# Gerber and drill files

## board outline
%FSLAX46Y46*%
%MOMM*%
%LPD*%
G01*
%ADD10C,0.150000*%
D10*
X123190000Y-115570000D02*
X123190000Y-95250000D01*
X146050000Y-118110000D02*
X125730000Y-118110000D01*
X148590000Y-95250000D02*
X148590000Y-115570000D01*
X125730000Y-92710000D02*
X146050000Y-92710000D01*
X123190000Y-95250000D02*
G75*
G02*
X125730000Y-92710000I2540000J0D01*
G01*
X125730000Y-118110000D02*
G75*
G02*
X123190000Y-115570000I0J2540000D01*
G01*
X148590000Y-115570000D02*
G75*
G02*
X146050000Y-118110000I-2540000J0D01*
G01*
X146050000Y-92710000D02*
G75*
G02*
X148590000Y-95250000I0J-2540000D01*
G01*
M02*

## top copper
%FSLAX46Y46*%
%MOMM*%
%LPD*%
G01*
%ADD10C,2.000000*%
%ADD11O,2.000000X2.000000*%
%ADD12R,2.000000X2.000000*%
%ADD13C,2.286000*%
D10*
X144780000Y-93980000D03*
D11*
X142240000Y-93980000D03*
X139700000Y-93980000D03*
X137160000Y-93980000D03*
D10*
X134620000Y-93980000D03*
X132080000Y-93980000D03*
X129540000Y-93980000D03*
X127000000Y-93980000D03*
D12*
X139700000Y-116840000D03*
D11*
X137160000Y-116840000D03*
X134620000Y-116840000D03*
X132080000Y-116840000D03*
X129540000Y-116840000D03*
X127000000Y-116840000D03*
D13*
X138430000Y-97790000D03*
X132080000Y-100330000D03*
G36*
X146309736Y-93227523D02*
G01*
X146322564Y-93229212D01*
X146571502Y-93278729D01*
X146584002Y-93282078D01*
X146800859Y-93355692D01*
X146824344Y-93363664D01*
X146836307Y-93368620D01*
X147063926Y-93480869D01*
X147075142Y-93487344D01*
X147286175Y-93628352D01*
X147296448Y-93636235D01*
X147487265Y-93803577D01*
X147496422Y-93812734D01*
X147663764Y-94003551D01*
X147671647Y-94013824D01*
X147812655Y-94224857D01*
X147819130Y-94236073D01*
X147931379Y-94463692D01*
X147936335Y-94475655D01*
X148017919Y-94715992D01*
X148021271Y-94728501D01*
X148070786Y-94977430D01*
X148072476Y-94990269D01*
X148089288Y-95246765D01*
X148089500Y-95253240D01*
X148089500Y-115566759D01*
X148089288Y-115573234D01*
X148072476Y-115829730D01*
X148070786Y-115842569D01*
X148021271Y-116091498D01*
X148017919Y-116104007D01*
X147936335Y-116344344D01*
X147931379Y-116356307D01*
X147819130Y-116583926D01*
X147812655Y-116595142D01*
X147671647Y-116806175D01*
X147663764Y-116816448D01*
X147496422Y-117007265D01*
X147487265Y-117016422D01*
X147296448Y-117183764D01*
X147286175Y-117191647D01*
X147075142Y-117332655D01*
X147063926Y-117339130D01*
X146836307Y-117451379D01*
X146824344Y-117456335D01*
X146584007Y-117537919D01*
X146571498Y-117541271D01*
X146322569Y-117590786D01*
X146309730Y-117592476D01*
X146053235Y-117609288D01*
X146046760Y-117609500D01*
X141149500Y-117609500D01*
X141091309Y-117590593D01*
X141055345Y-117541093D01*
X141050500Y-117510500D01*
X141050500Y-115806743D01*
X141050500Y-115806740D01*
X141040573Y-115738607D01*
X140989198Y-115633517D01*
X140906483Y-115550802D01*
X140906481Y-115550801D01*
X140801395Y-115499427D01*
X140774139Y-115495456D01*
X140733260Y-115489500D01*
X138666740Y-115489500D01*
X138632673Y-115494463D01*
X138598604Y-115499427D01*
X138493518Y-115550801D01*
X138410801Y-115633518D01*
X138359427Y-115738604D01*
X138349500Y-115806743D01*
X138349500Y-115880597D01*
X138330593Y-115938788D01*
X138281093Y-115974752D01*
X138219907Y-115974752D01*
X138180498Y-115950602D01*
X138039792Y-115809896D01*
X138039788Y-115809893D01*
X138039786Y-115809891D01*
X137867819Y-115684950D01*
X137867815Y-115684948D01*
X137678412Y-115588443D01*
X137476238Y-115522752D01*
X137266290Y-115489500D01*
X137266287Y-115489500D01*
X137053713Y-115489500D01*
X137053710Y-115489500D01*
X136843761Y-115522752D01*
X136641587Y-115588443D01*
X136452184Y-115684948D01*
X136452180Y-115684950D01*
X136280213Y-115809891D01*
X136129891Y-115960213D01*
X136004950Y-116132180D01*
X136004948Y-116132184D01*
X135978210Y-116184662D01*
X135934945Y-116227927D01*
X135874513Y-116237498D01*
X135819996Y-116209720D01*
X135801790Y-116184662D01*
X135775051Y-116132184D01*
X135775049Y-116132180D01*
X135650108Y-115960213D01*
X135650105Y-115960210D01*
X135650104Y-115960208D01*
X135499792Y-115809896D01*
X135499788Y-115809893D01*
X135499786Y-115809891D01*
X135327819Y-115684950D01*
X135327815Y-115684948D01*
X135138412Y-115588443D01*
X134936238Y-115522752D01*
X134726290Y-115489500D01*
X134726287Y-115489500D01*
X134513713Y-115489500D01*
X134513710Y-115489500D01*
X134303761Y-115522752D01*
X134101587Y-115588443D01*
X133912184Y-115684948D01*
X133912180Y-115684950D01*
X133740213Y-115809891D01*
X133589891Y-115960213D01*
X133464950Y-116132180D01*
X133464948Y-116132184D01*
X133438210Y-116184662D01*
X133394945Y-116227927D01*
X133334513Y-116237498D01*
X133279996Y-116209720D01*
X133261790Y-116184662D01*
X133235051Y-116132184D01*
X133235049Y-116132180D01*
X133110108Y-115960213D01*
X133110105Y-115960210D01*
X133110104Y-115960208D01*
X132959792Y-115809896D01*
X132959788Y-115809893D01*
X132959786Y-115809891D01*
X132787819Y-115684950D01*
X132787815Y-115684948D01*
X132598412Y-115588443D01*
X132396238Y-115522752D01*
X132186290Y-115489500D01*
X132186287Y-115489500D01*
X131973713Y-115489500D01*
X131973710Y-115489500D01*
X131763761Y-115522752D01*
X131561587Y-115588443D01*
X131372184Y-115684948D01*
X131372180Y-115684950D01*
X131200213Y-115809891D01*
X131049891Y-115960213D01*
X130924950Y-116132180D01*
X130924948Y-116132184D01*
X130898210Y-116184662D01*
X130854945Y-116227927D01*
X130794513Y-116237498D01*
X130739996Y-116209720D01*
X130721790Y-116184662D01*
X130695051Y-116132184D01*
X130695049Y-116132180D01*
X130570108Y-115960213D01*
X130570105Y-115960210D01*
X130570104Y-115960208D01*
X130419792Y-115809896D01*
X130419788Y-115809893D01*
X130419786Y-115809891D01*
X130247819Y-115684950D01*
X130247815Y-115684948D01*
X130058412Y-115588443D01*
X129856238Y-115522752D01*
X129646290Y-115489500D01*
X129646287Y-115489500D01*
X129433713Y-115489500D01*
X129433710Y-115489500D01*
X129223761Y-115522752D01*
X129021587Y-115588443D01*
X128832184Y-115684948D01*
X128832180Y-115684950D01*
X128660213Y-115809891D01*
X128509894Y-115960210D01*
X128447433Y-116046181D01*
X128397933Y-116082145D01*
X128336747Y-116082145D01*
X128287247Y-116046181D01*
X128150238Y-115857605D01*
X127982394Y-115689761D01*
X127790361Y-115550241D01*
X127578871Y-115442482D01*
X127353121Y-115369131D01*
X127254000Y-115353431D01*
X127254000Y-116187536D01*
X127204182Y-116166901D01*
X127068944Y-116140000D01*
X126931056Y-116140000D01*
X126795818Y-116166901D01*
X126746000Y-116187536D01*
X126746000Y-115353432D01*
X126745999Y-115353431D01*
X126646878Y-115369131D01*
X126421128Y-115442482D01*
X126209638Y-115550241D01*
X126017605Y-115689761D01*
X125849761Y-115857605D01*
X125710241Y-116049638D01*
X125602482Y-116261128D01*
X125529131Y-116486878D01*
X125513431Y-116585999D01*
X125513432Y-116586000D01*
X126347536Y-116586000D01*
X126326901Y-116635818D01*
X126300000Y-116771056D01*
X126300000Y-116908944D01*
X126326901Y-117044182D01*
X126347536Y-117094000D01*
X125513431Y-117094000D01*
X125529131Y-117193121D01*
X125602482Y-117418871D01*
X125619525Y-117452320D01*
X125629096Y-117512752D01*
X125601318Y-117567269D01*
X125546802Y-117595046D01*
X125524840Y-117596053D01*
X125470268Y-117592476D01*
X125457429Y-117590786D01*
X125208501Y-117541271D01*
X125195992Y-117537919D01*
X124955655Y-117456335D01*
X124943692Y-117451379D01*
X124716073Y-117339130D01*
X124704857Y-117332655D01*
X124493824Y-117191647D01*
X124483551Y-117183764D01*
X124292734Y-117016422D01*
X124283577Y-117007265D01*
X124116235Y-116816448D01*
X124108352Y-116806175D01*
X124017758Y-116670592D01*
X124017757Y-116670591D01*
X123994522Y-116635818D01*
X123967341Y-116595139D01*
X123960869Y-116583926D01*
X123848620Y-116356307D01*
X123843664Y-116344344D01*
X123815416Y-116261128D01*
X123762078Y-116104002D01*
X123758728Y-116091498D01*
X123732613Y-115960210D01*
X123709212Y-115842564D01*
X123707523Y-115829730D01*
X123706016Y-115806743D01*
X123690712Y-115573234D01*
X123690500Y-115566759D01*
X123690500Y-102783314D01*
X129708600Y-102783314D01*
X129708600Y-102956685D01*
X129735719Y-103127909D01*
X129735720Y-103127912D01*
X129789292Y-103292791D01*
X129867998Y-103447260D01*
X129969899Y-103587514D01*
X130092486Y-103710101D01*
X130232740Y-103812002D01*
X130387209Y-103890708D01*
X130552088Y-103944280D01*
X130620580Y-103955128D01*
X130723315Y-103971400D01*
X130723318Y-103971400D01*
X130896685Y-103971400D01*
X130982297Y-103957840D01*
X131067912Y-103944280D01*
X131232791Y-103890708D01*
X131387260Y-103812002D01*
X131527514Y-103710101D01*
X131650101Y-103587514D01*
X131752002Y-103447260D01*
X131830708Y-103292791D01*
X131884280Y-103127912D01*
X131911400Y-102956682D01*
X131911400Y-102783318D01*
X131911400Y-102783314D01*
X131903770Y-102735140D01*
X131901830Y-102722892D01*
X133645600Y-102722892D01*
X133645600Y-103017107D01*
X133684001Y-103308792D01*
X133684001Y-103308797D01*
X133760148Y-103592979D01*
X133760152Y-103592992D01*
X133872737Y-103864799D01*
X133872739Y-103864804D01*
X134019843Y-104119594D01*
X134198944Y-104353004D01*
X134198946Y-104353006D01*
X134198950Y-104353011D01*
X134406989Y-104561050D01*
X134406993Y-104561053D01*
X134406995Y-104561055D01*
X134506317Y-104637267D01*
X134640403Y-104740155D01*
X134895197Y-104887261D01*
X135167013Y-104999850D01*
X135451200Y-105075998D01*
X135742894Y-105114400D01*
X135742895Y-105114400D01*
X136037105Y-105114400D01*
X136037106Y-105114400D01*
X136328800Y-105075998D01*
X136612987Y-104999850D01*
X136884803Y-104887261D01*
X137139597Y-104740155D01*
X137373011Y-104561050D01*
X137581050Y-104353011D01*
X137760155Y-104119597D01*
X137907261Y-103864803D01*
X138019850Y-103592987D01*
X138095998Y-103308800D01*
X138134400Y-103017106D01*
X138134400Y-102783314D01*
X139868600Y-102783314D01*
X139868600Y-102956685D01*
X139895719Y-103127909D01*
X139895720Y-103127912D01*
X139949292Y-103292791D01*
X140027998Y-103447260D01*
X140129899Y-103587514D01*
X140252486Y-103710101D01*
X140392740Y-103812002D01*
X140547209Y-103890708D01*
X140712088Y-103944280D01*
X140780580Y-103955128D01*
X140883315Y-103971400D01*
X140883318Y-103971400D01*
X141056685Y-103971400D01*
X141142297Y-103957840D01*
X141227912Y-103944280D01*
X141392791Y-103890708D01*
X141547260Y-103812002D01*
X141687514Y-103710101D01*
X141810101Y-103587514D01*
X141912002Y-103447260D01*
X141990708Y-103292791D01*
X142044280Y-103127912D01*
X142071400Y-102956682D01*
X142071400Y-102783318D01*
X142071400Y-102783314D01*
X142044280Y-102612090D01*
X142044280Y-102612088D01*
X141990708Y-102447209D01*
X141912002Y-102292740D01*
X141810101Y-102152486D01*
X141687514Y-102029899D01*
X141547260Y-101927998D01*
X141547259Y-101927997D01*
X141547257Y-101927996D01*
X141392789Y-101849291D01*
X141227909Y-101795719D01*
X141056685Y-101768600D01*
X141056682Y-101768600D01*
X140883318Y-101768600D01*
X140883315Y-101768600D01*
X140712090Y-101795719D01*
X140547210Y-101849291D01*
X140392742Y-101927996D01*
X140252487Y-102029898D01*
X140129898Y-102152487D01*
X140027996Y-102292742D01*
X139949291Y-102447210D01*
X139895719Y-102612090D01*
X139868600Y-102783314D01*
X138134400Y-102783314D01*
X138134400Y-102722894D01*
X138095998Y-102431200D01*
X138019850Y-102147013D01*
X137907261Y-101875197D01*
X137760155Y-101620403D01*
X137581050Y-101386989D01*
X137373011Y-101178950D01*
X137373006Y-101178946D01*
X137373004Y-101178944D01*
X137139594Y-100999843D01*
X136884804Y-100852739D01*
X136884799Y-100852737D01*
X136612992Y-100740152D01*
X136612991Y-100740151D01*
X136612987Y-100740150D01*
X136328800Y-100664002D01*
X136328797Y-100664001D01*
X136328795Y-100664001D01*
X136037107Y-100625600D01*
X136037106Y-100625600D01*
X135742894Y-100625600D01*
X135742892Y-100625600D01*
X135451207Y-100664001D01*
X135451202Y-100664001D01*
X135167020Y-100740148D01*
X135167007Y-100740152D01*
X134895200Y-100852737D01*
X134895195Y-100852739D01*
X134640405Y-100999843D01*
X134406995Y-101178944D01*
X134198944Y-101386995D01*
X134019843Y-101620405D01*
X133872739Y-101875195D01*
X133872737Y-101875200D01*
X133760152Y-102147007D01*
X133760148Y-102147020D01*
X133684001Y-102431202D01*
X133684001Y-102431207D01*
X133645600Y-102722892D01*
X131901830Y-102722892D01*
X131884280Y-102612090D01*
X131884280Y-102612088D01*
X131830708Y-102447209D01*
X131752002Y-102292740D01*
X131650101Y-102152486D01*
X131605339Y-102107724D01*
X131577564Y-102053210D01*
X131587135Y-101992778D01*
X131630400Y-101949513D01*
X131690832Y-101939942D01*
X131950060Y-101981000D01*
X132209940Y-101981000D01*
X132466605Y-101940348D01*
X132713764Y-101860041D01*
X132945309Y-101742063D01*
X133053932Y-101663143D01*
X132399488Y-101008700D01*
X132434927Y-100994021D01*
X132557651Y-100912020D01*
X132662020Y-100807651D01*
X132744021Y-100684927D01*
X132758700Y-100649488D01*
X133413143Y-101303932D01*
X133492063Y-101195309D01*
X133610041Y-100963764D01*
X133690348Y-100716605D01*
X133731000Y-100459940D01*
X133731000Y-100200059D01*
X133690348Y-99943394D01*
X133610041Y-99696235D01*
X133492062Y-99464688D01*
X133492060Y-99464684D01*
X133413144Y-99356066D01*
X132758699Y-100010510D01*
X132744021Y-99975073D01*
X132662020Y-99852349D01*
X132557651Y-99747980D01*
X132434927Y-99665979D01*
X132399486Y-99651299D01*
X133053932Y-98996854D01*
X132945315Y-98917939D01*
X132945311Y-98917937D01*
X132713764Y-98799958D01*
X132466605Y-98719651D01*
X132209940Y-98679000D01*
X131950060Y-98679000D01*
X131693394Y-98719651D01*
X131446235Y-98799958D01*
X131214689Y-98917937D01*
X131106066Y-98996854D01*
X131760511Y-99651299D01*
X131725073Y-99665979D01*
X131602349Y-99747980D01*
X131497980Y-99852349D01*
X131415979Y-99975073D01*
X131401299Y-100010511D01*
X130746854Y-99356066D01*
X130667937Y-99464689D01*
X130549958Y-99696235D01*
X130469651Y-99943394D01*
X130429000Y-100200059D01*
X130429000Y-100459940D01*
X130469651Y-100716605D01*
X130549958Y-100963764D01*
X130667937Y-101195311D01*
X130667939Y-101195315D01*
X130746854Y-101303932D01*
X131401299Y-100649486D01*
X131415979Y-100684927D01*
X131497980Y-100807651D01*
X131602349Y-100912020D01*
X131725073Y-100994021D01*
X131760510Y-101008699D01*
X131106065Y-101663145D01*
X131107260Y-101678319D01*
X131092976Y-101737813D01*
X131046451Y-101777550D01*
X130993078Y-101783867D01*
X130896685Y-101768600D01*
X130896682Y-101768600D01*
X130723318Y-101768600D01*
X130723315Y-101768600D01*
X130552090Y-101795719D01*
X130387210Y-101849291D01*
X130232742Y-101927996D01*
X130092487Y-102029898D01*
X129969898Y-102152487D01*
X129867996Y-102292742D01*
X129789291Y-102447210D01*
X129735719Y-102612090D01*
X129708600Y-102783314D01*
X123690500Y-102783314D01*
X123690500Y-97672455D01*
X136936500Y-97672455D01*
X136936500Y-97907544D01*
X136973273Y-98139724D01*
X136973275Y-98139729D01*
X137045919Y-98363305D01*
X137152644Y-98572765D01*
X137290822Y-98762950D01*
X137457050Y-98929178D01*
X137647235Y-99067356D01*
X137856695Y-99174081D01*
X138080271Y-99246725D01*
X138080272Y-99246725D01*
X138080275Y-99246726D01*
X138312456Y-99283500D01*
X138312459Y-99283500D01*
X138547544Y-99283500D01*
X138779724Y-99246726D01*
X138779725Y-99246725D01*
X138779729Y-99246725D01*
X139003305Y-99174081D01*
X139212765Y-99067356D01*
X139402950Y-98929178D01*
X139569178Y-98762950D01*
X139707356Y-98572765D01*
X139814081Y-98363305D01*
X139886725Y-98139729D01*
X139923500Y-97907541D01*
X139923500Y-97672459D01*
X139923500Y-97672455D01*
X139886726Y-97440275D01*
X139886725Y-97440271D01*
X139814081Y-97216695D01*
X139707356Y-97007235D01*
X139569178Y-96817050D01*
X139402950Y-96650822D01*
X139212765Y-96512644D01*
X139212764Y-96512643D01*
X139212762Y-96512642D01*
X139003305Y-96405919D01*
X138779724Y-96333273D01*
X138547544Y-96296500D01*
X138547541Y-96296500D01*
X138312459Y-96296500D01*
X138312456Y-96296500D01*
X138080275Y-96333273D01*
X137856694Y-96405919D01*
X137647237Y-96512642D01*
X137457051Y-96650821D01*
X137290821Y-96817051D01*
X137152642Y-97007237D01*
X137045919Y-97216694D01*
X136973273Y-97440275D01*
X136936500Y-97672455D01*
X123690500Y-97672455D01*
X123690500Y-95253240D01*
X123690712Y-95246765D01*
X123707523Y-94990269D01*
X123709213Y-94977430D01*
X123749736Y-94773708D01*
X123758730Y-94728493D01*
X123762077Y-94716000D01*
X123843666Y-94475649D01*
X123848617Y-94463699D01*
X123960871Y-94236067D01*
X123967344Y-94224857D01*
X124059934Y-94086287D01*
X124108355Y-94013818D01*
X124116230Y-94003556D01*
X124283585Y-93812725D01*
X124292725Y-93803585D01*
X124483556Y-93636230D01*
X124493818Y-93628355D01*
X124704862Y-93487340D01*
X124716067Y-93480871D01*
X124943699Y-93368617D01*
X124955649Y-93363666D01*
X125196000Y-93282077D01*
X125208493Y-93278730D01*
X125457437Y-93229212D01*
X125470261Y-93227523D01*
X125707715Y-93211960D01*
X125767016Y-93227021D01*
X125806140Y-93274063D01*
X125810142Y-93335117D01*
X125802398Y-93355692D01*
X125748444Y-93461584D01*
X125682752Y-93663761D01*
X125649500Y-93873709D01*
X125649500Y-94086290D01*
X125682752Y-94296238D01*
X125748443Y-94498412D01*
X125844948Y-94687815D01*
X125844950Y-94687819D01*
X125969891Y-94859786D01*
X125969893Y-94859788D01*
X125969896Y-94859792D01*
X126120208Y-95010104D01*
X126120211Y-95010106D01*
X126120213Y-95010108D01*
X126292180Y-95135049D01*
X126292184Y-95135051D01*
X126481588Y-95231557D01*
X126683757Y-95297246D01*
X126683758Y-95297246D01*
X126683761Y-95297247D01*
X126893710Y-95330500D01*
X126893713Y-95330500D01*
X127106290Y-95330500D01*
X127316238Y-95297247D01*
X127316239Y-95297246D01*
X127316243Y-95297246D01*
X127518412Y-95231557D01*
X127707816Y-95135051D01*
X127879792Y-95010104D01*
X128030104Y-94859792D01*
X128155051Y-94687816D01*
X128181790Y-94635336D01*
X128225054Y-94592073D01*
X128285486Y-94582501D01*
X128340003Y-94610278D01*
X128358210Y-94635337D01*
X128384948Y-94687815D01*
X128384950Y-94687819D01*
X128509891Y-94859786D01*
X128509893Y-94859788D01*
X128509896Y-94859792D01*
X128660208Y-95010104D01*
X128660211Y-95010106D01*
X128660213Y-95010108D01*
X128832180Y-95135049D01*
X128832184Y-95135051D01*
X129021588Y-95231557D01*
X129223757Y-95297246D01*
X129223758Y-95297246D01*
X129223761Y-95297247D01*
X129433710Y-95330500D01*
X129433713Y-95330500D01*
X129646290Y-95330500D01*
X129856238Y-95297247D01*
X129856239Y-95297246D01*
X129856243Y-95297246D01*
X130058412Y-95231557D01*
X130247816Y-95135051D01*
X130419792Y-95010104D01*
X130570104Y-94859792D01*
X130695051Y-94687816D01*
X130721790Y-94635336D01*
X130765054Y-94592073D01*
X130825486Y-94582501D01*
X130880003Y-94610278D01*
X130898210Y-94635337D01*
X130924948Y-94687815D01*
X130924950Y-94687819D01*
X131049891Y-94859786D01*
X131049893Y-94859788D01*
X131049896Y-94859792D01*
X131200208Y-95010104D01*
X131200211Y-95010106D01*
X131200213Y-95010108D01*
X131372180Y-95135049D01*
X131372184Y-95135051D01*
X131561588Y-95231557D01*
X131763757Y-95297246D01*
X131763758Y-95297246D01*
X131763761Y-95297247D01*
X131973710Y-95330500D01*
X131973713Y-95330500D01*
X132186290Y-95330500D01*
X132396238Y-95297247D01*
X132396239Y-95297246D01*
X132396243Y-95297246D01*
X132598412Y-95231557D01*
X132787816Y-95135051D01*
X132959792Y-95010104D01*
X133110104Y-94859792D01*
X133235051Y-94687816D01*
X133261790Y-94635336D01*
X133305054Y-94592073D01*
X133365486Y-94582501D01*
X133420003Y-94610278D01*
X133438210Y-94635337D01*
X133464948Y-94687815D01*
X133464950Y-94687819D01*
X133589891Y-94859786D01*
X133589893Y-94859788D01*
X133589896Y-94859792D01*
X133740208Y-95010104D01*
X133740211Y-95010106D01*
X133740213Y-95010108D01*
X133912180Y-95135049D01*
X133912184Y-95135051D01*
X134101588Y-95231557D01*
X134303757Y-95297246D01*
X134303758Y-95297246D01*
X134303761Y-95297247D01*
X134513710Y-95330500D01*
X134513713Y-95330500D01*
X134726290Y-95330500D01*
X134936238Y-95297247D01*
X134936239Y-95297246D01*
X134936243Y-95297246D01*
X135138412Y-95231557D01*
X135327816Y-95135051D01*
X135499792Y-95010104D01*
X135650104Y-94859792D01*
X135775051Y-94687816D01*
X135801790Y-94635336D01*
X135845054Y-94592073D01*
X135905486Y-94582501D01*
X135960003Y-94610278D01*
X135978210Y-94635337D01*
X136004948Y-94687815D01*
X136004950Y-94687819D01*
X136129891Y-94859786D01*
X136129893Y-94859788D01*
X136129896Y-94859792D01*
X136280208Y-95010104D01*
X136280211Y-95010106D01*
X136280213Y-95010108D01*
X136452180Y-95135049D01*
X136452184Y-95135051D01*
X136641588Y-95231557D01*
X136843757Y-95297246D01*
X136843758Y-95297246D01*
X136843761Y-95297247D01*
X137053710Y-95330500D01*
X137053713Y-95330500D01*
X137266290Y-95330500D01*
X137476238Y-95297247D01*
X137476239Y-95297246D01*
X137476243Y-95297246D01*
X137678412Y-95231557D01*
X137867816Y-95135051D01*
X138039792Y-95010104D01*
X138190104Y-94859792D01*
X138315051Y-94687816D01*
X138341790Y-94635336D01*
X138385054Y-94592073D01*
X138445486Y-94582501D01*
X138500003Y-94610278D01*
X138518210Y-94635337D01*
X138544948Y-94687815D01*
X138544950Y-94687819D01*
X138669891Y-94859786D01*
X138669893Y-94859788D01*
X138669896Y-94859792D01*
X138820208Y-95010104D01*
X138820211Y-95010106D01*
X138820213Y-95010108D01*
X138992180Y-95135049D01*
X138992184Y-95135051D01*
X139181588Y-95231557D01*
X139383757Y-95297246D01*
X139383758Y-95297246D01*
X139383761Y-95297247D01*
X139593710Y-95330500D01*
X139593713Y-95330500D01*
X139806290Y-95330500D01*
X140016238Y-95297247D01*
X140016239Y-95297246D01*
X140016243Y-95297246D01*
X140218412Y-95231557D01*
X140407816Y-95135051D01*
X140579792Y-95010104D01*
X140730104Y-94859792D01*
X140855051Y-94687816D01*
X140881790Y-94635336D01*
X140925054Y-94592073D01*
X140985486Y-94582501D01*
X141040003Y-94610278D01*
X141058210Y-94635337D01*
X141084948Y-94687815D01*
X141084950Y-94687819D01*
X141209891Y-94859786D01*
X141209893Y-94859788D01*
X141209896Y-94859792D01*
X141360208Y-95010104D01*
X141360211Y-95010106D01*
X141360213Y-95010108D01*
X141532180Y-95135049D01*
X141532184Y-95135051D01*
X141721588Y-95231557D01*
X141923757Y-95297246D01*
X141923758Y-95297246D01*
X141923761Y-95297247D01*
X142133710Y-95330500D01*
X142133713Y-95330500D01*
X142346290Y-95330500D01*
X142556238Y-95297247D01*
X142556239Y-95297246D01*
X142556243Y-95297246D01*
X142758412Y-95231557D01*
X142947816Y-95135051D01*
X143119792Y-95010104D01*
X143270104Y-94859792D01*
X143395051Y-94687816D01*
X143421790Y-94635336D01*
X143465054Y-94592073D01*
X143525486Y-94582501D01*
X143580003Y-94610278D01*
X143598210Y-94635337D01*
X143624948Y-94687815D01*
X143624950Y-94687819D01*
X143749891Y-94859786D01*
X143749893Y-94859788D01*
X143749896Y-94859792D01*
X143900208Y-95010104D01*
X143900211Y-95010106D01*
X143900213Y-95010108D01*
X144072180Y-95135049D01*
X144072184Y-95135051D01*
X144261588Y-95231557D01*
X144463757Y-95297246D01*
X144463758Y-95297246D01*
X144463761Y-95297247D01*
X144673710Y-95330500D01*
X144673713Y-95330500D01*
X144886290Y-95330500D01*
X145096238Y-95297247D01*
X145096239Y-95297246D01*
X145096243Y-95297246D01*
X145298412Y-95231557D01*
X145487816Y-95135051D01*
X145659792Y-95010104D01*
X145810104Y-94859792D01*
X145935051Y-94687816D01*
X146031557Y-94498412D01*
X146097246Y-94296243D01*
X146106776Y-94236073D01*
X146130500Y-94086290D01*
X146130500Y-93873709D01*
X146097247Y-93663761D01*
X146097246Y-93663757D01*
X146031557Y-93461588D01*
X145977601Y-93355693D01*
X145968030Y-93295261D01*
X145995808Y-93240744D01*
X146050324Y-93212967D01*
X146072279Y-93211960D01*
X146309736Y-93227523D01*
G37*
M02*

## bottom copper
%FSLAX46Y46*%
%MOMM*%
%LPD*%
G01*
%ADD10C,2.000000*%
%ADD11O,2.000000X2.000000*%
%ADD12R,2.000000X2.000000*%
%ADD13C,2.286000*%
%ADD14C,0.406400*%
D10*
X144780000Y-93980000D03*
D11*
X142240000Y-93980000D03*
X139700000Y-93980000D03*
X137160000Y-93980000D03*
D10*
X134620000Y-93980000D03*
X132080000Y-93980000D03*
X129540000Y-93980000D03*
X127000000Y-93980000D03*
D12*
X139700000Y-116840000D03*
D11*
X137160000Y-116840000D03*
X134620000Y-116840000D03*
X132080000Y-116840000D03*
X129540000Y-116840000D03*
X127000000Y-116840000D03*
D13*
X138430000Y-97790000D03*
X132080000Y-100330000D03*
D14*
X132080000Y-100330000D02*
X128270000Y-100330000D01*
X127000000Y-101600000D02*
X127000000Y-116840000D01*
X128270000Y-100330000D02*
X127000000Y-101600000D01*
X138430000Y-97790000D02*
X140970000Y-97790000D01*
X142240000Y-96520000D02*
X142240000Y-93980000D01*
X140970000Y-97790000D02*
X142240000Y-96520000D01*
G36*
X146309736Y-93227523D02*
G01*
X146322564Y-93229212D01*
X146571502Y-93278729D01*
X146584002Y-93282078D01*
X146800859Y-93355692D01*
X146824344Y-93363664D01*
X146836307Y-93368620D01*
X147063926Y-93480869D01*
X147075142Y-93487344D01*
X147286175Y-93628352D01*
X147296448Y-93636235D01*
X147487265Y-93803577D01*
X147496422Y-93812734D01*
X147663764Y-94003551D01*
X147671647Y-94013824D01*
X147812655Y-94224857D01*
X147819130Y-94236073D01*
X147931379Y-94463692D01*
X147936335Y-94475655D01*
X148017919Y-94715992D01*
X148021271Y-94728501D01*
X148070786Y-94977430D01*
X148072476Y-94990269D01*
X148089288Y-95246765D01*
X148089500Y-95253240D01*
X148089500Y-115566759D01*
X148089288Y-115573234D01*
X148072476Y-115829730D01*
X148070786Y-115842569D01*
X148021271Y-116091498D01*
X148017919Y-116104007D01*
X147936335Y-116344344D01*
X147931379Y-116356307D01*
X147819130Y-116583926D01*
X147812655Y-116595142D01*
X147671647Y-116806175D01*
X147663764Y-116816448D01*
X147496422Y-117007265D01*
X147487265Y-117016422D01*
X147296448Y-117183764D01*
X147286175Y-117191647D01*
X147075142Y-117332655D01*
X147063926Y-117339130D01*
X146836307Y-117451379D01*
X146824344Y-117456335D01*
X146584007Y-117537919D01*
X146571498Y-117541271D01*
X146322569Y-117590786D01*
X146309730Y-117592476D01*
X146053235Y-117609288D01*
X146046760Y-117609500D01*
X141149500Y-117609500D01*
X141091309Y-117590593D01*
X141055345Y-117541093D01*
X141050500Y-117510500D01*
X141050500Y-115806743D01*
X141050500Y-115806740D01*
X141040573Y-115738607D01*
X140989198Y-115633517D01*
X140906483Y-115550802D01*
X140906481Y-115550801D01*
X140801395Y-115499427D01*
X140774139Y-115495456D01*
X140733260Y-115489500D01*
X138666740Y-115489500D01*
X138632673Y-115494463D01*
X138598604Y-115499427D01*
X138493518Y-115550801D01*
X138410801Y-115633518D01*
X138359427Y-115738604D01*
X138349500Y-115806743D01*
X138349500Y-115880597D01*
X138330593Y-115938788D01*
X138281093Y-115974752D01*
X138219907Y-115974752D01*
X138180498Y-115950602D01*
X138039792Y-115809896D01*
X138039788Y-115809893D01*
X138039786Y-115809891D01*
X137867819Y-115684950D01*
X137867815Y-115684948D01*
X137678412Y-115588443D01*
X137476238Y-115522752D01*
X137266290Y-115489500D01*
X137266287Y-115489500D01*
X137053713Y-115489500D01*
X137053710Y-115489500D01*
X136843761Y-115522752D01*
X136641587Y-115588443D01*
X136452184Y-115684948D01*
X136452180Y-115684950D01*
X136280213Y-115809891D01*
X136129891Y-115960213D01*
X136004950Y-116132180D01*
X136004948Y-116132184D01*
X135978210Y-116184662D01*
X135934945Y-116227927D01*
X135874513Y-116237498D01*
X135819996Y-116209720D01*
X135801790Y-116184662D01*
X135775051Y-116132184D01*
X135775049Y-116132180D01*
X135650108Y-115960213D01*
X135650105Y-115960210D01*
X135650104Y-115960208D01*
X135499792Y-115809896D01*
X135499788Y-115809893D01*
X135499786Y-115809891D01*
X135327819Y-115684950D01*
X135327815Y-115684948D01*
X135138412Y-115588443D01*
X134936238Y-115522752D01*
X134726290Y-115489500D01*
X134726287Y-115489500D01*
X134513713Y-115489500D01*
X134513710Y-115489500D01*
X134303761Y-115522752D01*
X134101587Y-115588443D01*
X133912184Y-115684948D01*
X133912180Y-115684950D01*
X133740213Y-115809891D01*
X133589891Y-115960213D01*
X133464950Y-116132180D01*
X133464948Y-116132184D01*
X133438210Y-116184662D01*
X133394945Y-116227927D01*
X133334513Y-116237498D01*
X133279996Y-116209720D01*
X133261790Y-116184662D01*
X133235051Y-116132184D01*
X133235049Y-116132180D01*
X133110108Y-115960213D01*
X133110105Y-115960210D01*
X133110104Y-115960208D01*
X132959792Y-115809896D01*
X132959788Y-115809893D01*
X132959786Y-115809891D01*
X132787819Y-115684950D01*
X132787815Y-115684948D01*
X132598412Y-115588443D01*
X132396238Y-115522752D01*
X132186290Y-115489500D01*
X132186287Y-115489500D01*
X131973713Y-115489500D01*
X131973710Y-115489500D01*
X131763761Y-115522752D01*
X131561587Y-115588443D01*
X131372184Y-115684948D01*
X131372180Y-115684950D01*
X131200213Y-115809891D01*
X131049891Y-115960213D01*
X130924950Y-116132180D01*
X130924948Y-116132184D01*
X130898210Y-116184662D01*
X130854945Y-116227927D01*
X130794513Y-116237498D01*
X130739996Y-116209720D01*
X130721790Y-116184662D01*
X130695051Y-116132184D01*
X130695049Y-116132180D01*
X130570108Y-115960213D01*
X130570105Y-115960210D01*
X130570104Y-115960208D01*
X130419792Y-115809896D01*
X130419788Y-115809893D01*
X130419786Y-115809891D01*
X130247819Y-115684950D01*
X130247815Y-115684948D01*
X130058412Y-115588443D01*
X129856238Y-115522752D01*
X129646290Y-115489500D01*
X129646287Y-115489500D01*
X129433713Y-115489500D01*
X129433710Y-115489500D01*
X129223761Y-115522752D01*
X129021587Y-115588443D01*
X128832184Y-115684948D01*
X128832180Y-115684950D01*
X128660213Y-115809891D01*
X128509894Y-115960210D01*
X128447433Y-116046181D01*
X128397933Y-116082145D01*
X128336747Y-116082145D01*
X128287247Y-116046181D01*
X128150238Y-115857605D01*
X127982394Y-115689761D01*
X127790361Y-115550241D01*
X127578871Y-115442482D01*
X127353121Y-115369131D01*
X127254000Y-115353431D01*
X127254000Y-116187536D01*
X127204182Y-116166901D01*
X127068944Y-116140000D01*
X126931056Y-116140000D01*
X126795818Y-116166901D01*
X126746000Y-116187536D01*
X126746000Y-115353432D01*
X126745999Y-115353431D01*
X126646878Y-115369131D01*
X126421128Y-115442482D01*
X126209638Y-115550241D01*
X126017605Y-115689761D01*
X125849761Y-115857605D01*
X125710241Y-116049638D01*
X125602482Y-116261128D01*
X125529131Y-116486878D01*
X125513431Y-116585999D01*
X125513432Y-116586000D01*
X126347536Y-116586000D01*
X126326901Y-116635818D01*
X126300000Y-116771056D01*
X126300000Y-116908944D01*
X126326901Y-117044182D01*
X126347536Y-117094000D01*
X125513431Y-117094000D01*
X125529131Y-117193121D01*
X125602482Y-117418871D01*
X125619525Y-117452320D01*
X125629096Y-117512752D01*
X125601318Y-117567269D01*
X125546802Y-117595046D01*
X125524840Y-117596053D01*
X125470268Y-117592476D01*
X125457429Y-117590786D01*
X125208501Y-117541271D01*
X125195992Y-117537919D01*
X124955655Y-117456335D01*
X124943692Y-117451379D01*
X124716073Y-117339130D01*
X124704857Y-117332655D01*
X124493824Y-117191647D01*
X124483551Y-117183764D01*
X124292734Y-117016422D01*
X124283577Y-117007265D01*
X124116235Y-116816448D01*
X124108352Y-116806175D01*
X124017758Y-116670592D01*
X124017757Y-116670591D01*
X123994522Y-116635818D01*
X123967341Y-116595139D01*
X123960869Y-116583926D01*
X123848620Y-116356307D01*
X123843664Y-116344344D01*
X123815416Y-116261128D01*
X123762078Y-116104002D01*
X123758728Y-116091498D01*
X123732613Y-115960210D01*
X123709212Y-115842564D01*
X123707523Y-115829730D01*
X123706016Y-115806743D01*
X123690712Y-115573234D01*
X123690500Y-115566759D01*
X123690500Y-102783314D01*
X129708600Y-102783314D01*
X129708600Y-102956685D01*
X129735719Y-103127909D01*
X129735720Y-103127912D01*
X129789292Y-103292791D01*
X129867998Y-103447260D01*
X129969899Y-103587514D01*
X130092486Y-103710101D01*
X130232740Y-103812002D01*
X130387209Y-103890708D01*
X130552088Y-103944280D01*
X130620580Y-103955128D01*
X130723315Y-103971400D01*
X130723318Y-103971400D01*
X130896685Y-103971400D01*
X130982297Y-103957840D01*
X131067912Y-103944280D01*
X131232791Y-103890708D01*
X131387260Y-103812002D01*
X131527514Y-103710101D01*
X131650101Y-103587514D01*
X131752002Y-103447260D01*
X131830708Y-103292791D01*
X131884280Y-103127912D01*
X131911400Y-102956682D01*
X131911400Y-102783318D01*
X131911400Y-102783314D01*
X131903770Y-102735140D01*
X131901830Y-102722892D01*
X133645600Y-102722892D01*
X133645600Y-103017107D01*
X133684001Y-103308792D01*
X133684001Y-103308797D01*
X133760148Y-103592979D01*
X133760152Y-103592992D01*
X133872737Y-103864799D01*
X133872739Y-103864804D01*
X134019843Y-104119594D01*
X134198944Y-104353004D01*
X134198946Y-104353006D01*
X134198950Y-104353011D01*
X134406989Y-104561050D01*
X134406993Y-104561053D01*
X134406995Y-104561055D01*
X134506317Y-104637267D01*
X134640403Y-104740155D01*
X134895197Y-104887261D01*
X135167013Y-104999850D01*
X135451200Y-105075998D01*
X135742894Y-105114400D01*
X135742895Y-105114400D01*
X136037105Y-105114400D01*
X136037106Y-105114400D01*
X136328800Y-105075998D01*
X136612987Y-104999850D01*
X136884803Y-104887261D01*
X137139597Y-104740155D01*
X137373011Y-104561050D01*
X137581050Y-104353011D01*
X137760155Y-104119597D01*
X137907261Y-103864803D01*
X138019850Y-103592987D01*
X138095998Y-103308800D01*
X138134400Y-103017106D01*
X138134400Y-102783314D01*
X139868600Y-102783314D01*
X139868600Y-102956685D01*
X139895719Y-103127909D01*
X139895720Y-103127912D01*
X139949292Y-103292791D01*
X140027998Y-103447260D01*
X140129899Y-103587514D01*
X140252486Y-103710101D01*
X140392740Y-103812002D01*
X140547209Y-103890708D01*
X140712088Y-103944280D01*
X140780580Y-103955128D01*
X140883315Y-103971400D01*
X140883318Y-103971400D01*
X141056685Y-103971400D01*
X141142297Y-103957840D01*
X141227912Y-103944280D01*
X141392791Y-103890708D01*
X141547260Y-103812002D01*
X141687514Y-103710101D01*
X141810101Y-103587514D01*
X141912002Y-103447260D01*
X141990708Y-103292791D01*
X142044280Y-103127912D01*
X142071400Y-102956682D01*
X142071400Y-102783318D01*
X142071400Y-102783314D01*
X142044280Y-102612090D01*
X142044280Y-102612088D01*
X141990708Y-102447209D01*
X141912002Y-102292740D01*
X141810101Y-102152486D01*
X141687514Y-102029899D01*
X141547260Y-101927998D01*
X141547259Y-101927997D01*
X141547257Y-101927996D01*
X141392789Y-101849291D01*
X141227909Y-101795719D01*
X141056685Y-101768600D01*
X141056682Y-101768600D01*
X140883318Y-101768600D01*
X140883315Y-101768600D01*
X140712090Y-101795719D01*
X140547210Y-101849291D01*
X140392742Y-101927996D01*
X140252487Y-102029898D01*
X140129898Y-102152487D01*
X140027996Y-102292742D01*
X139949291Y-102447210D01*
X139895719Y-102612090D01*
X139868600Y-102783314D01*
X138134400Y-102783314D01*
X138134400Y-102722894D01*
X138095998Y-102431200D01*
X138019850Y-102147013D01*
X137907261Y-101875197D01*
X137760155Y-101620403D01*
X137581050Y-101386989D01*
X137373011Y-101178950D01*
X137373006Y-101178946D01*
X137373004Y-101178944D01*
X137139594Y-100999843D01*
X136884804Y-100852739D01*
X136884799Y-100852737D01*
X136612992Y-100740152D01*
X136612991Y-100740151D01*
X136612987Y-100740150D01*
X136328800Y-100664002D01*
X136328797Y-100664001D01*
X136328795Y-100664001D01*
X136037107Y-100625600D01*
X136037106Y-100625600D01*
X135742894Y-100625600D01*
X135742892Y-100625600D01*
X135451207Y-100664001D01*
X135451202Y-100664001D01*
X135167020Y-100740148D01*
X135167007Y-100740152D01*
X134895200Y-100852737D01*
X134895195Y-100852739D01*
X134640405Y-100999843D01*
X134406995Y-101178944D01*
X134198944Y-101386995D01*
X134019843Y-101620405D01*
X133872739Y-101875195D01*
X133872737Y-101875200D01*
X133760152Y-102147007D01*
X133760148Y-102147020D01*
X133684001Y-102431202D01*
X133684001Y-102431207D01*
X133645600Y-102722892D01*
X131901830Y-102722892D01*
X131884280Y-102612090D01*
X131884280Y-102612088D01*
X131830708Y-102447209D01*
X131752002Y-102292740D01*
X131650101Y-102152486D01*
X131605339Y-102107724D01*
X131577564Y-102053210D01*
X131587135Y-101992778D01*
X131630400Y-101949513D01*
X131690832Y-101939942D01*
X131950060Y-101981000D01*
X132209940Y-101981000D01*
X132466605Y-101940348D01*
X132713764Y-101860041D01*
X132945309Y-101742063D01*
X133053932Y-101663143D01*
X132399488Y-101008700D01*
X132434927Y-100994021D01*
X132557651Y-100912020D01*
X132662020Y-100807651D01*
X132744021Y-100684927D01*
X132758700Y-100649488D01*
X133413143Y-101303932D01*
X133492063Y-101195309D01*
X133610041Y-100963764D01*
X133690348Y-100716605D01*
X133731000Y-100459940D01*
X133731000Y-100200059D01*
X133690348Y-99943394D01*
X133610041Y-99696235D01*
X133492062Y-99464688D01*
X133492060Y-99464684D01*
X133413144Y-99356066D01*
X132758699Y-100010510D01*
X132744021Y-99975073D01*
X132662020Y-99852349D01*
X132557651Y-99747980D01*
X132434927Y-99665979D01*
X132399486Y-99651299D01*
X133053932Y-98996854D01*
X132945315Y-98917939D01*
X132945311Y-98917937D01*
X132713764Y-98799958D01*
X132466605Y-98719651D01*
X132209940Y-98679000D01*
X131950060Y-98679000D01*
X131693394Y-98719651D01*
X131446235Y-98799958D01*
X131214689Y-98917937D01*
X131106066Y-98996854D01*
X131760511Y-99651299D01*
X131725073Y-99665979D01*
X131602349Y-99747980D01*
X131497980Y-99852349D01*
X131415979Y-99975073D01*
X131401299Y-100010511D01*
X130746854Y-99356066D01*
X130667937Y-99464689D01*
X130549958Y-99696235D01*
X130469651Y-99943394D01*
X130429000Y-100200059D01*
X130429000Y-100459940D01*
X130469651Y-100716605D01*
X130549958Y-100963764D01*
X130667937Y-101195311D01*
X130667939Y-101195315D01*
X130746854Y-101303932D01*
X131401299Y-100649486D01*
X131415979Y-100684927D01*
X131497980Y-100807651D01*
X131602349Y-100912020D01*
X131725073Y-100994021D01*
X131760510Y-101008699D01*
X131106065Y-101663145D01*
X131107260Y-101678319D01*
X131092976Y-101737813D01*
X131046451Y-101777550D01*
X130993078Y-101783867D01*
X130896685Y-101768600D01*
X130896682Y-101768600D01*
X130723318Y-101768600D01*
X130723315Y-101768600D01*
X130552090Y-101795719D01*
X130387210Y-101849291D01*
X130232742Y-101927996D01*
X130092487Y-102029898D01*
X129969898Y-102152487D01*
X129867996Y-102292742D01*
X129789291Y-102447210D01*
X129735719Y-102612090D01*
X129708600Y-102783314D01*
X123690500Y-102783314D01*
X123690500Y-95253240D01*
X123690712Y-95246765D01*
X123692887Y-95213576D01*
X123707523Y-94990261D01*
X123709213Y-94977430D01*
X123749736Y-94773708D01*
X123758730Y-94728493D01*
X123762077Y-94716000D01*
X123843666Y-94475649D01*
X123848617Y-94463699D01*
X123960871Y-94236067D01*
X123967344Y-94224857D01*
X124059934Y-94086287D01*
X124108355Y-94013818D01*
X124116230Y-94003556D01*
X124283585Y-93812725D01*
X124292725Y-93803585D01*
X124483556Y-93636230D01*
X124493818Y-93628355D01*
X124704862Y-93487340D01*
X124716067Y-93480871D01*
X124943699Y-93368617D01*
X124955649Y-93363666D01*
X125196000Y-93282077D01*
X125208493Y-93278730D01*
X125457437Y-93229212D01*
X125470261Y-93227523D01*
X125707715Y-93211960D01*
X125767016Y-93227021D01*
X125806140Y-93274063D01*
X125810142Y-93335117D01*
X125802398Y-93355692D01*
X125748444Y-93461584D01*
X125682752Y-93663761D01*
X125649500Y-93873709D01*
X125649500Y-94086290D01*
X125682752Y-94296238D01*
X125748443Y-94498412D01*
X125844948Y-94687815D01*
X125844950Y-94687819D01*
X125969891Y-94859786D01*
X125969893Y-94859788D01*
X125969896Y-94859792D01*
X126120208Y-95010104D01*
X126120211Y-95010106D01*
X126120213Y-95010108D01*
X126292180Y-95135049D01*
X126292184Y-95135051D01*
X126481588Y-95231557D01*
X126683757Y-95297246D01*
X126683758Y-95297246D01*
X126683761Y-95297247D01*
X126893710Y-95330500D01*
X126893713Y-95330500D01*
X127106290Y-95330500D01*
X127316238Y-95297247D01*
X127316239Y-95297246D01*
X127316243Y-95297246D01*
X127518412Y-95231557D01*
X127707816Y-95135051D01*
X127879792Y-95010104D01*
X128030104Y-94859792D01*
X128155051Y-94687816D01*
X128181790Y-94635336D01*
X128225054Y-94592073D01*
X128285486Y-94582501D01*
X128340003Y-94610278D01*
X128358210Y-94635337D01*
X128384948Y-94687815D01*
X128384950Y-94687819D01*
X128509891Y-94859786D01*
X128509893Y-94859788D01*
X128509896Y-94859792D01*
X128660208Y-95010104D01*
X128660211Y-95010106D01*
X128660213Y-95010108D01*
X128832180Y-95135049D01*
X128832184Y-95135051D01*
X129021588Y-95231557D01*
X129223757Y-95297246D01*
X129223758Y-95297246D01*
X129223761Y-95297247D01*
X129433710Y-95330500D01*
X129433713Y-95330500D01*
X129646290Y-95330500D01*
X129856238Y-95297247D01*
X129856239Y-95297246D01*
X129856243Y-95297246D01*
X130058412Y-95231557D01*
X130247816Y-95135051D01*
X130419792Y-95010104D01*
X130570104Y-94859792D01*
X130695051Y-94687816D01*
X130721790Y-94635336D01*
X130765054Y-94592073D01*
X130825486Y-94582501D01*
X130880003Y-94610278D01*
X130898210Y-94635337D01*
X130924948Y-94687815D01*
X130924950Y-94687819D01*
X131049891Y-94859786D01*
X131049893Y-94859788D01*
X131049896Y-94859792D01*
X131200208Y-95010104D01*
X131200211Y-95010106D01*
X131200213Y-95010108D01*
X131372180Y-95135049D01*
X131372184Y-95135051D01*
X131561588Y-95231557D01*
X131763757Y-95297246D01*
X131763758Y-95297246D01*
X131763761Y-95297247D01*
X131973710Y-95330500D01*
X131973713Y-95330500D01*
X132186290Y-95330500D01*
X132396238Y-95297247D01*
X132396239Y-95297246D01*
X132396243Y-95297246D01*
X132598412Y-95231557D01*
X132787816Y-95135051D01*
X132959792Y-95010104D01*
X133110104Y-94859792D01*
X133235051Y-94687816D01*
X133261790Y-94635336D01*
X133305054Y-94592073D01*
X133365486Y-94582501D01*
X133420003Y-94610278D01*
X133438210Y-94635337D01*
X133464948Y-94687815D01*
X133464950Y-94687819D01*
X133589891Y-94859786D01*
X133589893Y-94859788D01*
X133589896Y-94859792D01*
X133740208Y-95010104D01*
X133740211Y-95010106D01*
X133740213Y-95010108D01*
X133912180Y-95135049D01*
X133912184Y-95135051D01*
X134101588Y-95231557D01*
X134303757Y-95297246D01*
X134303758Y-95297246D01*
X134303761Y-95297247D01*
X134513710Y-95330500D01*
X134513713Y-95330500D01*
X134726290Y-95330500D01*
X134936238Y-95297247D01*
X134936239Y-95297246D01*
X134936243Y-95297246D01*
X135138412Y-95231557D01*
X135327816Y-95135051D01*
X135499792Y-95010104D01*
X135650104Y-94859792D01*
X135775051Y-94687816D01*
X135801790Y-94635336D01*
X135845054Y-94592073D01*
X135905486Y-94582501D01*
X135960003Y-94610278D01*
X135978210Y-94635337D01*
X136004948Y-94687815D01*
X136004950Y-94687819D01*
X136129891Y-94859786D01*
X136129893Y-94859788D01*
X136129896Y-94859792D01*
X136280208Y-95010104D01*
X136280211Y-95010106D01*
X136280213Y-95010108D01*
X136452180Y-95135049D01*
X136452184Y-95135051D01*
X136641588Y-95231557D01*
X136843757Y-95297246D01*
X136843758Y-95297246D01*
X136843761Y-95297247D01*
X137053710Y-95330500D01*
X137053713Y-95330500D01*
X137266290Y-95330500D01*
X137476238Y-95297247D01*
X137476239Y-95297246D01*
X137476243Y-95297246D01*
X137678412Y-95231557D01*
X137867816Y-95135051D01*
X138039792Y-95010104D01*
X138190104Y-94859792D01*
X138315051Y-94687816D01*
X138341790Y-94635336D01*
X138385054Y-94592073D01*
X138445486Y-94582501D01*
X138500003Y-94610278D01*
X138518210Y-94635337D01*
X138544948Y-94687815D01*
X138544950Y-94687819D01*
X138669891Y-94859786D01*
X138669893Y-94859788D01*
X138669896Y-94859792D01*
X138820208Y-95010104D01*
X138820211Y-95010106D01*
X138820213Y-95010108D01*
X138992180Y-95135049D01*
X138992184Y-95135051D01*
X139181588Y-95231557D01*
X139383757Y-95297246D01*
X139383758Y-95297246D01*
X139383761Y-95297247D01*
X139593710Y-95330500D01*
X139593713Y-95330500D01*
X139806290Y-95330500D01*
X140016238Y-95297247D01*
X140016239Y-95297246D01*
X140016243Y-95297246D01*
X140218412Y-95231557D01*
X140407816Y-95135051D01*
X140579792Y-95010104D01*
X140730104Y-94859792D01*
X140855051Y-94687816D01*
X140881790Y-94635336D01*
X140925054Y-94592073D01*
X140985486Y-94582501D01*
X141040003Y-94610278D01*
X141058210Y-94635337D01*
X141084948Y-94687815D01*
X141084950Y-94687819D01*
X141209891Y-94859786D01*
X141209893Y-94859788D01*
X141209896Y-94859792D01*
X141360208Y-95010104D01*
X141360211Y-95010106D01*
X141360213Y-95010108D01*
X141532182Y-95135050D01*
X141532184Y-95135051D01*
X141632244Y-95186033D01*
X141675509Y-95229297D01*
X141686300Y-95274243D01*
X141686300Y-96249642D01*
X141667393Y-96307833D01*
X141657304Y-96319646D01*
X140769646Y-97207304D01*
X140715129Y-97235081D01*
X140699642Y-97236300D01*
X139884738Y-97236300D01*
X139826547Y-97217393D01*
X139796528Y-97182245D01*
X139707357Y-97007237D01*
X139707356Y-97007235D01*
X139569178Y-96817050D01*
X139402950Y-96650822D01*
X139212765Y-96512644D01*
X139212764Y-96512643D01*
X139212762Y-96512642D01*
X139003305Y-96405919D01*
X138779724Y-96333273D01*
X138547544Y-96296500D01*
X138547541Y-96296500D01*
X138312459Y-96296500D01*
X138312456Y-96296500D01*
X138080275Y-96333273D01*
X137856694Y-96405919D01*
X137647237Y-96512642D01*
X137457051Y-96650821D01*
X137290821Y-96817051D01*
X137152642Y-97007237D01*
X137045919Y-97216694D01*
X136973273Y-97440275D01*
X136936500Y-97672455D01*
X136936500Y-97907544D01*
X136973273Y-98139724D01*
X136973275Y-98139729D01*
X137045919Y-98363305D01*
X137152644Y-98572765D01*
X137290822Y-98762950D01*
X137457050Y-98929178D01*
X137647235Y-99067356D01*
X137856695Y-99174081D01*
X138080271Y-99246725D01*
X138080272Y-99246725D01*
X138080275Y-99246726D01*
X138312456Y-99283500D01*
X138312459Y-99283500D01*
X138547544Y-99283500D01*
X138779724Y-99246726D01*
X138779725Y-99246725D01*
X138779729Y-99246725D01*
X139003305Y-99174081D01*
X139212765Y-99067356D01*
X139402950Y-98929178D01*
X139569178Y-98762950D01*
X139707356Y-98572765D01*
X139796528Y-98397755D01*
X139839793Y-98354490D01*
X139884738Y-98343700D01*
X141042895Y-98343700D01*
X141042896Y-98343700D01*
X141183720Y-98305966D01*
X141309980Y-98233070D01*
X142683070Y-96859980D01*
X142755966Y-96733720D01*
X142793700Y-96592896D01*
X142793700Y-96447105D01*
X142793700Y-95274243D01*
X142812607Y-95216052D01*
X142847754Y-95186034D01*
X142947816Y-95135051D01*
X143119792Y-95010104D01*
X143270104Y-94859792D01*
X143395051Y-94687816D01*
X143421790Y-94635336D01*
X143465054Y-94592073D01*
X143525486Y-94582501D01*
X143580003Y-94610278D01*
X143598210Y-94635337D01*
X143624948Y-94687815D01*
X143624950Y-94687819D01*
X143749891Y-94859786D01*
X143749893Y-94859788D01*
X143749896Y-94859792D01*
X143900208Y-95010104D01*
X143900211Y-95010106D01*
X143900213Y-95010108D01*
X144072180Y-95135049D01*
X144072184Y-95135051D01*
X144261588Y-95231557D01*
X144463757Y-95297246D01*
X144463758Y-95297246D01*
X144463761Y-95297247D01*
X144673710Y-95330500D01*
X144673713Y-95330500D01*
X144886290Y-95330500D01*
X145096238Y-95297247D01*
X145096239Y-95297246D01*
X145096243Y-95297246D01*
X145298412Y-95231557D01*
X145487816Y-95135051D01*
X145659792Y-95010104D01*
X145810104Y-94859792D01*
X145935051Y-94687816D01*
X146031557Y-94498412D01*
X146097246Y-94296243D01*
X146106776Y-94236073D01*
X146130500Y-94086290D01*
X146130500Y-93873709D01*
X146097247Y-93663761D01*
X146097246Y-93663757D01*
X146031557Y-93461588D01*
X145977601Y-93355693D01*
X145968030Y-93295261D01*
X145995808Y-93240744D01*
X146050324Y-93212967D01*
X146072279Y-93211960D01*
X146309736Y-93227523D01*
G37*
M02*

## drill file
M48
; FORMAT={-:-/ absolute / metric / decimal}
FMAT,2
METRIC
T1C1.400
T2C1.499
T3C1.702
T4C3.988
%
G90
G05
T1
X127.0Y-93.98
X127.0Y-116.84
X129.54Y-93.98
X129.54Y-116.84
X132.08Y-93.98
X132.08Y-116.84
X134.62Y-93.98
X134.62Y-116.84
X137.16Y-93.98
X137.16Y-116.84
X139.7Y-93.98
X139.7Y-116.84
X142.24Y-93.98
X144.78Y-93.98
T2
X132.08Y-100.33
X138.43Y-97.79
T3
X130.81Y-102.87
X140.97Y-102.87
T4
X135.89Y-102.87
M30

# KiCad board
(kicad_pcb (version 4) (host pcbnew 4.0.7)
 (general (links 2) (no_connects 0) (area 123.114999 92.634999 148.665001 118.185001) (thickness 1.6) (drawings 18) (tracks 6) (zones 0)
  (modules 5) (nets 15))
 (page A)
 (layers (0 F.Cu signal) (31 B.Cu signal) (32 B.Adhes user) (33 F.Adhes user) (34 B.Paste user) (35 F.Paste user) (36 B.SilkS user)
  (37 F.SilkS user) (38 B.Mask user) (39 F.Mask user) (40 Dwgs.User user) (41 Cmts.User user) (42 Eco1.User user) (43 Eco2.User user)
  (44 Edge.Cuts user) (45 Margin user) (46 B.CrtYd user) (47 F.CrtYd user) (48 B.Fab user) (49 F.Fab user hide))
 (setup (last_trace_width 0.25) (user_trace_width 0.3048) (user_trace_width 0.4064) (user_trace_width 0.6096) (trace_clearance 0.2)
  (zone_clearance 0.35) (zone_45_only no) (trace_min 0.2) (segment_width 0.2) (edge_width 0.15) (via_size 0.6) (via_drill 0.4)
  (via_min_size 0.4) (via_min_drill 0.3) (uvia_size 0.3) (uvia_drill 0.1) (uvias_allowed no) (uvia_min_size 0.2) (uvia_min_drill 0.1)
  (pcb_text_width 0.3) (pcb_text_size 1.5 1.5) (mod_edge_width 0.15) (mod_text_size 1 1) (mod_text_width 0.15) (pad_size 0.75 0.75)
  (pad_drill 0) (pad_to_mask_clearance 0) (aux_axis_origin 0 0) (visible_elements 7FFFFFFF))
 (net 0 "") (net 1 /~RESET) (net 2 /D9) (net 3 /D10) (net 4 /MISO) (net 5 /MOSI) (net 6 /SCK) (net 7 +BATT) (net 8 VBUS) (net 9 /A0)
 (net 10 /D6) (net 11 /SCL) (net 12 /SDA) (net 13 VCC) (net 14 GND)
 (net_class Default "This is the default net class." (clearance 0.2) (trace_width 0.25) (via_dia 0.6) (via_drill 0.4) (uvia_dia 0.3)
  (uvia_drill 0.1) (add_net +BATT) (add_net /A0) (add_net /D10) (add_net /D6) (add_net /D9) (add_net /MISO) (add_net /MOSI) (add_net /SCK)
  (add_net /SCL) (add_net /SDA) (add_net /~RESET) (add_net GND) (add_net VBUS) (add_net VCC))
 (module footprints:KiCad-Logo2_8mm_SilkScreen (layer B.Cu) (at 139.192 109.347 180)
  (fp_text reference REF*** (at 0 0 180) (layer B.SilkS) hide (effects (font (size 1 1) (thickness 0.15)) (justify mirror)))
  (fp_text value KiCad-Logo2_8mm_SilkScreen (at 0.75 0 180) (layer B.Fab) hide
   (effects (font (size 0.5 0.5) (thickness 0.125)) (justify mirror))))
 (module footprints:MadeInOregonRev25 (layer F.Cu) (at 127 108.966)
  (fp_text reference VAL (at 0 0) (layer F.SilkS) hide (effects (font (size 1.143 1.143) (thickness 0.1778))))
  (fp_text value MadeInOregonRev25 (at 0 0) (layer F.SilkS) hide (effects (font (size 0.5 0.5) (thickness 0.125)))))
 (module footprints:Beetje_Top (layer F.Cu) (at 144.78 93.98 270)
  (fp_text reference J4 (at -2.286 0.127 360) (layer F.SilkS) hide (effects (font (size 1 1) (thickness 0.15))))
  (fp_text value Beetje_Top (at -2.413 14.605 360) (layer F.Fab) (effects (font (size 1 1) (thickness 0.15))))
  (pad 1 thru_hole circle (at 0 0 270) (size 2 2) (drill 1.4) (layers *.Cu *.Mask) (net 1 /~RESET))
  (pad 2 thru_hole oval (at 0 2.54 270) (size 2 2) (drill 1.4) (layers *.Cu *.Mask) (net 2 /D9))
  (pad 3 thru_hole oval (at 0 5.08 270) (size 2 2) (drill 1.4) (layers *.Cu *.Mask) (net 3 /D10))
  (pad 4 thru_hole oval (at 0 7.62 270) (size 2 2) (drill 1.4) (layers *.Cu *.Mask) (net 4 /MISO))
  (pad 5 thru_hole circle (at 0 10.16 270) (size 2 2) (drill 1.4) (layers *.Cu *.Mask) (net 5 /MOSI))
  (pad 6 thru_hole circle (at 0 12.7 270) (size 2 2) (drill 1.4) (layers *.Cu *.Mask) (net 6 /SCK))
  (pad 7 thru_hole circle (at 0 15.24 270) (size 2 2) (drill 1.4) (layers *.Cu *.Mask) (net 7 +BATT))
  (pad 8 thru_hole circle (at 0 17.78 270) (size 2 2) (drill 1.4) (layers *.Cu *.Mask) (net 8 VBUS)))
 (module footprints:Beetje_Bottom (layer F.Cu) (at 139.7 116.84 270)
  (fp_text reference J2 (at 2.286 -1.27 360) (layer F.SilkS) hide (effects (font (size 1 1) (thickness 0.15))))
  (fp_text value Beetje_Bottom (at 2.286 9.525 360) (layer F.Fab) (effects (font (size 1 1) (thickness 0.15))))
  (pad 1 thru_hole rect (at 0 0 270) (size 2 2) (drill 1.4) (layers *.Cu *.Mask) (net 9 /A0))
  (pad 2 thru_hole oval (at 0 2.54 270) (size 2 2) (drill 1.4) (layers *.Cu *.Mask) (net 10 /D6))
  (pad 3 thru_hole oval (at 0 5.08 270) (size 2 2) (drill 1.4) (layers *.Cu *.Mask) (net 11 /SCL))
  (pad 4 thru_hole oval (at 0 7.62 270) (size 2 2) (drill 1.4) (layers *.Cu *.Mask) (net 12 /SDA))
  (pad 5 thru_hole oval (at 0 10.16 270) (size 2 2) (drill 1.4) (layers *.Cu *.Mask) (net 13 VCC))
  (pad 6 thru_hole oval (at 0 12.7 270) (size 2 2) (drill 1.4) (layers *.Cu *.Mask) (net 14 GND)))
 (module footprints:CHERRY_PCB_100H (layer F.Cu) (at 135.89 102.87)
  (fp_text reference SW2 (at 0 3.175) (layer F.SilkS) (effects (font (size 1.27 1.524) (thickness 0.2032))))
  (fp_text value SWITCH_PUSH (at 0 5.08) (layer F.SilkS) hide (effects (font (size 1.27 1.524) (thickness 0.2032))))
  (pad 1 thru_hole circle (at 2.54 -5.08) (size 2.286 2.286) (drill 1.4986) (layers *.Cu *.SilkS *.Mask) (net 2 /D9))
  (pad 2 thru_hole circle (at -3.81 -2.54) (size 2.286 2.286) (drill 1.4986) (layers *.Cu *.SilkS *.Mask) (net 14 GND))
  (pad HOLE np_thru_hole circle (at 0 0) (size 3.9878 3.9878) (drill 3.9878) (layers *.Cu))
  (pad HOLE np_thru_hole circle (at -5.08 0) (size 1.7018 1.7018) (drill 1.7018) (layers *.Cu))
  (pad HOLE np_thru_hole circle (at 5.08 0) (size 1.7018 1.7018) (drill 1.7018) (layers *.Cu)))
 (gr_line (start 123.19 115.57) (end 123.19 95.25) (angle 90) (layer Edge.Cuts) (width 0.15))
 (gr_line (start 146.05 118.11) (end 125.73 118.11) (angle 90) (layer Edge.Cuts) (width 0.15))
 (gr_line (start 148.59 95.25) (end 148.59 115.57) (angle 90) (layer Edge.Cuts) (width 0.15))
 (gr_line (start 125.73 92.71) (end 146.05 92.71) (angle 90) (layer Edge.Cuts) (width 0.15))
 (gr_arc (start 125.73 95.25) (end 123.19 95.25) (angle 90) (layer Edge.Cuts) (width 0.15))
 (gr_arc (start 125.73 115.57) (end 125.73 118.11) (angle 90) (layer Edge.Cuts) (width 0.15))
 (gr_arc (start 146.05 115.57) (end 148.59 115.57) (angle 90) (layer Edge.Cuts) (width 0.15))
 (gr_arc (start 146.05 95.25) (end 146.05 92.71) (angle 90) (layer Edge.Cuts) (width 0.15))
 (segment (start 132.08 100.33) (end 128.27 100.33) (width 0.4064) (layer B.Cu) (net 14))
 (segment (start 127 101.6) (end 127 116.84) (width 0.4064) (layer B.Cu) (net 14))
 (segment (start 128.27 100.33) (end 127 101.6) (width 0.4064) (layer B.Cu) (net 14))
 (segment (start 138.43 97.79) (end 140.97 97.79) (width 0.4064) (layer B.Cu) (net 2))
 (segment (start 142.24 96.52) (end 142.24 93.98) (width 0.4064) (layer B.Cu) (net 2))
 (segment (start 140.97 97.79) (end 142.24 96.52) (width 0.4064) (layer B.Cu) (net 2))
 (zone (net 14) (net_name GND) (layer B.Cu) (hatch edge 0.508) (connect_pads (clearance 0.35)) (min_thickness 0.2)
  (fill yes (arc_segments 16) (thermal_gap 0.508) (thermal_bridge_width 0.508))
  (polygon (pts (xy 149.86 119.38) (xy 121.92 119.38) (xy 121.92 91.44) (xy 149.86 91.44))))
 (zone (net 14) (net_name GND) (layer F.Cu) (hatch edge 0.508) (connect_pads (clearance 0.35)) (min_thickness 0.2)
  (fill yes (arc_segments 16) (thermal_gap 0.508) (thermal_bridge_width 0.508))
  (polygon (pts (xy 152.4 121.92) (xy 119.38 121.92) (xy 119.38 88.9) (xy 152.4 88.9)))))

